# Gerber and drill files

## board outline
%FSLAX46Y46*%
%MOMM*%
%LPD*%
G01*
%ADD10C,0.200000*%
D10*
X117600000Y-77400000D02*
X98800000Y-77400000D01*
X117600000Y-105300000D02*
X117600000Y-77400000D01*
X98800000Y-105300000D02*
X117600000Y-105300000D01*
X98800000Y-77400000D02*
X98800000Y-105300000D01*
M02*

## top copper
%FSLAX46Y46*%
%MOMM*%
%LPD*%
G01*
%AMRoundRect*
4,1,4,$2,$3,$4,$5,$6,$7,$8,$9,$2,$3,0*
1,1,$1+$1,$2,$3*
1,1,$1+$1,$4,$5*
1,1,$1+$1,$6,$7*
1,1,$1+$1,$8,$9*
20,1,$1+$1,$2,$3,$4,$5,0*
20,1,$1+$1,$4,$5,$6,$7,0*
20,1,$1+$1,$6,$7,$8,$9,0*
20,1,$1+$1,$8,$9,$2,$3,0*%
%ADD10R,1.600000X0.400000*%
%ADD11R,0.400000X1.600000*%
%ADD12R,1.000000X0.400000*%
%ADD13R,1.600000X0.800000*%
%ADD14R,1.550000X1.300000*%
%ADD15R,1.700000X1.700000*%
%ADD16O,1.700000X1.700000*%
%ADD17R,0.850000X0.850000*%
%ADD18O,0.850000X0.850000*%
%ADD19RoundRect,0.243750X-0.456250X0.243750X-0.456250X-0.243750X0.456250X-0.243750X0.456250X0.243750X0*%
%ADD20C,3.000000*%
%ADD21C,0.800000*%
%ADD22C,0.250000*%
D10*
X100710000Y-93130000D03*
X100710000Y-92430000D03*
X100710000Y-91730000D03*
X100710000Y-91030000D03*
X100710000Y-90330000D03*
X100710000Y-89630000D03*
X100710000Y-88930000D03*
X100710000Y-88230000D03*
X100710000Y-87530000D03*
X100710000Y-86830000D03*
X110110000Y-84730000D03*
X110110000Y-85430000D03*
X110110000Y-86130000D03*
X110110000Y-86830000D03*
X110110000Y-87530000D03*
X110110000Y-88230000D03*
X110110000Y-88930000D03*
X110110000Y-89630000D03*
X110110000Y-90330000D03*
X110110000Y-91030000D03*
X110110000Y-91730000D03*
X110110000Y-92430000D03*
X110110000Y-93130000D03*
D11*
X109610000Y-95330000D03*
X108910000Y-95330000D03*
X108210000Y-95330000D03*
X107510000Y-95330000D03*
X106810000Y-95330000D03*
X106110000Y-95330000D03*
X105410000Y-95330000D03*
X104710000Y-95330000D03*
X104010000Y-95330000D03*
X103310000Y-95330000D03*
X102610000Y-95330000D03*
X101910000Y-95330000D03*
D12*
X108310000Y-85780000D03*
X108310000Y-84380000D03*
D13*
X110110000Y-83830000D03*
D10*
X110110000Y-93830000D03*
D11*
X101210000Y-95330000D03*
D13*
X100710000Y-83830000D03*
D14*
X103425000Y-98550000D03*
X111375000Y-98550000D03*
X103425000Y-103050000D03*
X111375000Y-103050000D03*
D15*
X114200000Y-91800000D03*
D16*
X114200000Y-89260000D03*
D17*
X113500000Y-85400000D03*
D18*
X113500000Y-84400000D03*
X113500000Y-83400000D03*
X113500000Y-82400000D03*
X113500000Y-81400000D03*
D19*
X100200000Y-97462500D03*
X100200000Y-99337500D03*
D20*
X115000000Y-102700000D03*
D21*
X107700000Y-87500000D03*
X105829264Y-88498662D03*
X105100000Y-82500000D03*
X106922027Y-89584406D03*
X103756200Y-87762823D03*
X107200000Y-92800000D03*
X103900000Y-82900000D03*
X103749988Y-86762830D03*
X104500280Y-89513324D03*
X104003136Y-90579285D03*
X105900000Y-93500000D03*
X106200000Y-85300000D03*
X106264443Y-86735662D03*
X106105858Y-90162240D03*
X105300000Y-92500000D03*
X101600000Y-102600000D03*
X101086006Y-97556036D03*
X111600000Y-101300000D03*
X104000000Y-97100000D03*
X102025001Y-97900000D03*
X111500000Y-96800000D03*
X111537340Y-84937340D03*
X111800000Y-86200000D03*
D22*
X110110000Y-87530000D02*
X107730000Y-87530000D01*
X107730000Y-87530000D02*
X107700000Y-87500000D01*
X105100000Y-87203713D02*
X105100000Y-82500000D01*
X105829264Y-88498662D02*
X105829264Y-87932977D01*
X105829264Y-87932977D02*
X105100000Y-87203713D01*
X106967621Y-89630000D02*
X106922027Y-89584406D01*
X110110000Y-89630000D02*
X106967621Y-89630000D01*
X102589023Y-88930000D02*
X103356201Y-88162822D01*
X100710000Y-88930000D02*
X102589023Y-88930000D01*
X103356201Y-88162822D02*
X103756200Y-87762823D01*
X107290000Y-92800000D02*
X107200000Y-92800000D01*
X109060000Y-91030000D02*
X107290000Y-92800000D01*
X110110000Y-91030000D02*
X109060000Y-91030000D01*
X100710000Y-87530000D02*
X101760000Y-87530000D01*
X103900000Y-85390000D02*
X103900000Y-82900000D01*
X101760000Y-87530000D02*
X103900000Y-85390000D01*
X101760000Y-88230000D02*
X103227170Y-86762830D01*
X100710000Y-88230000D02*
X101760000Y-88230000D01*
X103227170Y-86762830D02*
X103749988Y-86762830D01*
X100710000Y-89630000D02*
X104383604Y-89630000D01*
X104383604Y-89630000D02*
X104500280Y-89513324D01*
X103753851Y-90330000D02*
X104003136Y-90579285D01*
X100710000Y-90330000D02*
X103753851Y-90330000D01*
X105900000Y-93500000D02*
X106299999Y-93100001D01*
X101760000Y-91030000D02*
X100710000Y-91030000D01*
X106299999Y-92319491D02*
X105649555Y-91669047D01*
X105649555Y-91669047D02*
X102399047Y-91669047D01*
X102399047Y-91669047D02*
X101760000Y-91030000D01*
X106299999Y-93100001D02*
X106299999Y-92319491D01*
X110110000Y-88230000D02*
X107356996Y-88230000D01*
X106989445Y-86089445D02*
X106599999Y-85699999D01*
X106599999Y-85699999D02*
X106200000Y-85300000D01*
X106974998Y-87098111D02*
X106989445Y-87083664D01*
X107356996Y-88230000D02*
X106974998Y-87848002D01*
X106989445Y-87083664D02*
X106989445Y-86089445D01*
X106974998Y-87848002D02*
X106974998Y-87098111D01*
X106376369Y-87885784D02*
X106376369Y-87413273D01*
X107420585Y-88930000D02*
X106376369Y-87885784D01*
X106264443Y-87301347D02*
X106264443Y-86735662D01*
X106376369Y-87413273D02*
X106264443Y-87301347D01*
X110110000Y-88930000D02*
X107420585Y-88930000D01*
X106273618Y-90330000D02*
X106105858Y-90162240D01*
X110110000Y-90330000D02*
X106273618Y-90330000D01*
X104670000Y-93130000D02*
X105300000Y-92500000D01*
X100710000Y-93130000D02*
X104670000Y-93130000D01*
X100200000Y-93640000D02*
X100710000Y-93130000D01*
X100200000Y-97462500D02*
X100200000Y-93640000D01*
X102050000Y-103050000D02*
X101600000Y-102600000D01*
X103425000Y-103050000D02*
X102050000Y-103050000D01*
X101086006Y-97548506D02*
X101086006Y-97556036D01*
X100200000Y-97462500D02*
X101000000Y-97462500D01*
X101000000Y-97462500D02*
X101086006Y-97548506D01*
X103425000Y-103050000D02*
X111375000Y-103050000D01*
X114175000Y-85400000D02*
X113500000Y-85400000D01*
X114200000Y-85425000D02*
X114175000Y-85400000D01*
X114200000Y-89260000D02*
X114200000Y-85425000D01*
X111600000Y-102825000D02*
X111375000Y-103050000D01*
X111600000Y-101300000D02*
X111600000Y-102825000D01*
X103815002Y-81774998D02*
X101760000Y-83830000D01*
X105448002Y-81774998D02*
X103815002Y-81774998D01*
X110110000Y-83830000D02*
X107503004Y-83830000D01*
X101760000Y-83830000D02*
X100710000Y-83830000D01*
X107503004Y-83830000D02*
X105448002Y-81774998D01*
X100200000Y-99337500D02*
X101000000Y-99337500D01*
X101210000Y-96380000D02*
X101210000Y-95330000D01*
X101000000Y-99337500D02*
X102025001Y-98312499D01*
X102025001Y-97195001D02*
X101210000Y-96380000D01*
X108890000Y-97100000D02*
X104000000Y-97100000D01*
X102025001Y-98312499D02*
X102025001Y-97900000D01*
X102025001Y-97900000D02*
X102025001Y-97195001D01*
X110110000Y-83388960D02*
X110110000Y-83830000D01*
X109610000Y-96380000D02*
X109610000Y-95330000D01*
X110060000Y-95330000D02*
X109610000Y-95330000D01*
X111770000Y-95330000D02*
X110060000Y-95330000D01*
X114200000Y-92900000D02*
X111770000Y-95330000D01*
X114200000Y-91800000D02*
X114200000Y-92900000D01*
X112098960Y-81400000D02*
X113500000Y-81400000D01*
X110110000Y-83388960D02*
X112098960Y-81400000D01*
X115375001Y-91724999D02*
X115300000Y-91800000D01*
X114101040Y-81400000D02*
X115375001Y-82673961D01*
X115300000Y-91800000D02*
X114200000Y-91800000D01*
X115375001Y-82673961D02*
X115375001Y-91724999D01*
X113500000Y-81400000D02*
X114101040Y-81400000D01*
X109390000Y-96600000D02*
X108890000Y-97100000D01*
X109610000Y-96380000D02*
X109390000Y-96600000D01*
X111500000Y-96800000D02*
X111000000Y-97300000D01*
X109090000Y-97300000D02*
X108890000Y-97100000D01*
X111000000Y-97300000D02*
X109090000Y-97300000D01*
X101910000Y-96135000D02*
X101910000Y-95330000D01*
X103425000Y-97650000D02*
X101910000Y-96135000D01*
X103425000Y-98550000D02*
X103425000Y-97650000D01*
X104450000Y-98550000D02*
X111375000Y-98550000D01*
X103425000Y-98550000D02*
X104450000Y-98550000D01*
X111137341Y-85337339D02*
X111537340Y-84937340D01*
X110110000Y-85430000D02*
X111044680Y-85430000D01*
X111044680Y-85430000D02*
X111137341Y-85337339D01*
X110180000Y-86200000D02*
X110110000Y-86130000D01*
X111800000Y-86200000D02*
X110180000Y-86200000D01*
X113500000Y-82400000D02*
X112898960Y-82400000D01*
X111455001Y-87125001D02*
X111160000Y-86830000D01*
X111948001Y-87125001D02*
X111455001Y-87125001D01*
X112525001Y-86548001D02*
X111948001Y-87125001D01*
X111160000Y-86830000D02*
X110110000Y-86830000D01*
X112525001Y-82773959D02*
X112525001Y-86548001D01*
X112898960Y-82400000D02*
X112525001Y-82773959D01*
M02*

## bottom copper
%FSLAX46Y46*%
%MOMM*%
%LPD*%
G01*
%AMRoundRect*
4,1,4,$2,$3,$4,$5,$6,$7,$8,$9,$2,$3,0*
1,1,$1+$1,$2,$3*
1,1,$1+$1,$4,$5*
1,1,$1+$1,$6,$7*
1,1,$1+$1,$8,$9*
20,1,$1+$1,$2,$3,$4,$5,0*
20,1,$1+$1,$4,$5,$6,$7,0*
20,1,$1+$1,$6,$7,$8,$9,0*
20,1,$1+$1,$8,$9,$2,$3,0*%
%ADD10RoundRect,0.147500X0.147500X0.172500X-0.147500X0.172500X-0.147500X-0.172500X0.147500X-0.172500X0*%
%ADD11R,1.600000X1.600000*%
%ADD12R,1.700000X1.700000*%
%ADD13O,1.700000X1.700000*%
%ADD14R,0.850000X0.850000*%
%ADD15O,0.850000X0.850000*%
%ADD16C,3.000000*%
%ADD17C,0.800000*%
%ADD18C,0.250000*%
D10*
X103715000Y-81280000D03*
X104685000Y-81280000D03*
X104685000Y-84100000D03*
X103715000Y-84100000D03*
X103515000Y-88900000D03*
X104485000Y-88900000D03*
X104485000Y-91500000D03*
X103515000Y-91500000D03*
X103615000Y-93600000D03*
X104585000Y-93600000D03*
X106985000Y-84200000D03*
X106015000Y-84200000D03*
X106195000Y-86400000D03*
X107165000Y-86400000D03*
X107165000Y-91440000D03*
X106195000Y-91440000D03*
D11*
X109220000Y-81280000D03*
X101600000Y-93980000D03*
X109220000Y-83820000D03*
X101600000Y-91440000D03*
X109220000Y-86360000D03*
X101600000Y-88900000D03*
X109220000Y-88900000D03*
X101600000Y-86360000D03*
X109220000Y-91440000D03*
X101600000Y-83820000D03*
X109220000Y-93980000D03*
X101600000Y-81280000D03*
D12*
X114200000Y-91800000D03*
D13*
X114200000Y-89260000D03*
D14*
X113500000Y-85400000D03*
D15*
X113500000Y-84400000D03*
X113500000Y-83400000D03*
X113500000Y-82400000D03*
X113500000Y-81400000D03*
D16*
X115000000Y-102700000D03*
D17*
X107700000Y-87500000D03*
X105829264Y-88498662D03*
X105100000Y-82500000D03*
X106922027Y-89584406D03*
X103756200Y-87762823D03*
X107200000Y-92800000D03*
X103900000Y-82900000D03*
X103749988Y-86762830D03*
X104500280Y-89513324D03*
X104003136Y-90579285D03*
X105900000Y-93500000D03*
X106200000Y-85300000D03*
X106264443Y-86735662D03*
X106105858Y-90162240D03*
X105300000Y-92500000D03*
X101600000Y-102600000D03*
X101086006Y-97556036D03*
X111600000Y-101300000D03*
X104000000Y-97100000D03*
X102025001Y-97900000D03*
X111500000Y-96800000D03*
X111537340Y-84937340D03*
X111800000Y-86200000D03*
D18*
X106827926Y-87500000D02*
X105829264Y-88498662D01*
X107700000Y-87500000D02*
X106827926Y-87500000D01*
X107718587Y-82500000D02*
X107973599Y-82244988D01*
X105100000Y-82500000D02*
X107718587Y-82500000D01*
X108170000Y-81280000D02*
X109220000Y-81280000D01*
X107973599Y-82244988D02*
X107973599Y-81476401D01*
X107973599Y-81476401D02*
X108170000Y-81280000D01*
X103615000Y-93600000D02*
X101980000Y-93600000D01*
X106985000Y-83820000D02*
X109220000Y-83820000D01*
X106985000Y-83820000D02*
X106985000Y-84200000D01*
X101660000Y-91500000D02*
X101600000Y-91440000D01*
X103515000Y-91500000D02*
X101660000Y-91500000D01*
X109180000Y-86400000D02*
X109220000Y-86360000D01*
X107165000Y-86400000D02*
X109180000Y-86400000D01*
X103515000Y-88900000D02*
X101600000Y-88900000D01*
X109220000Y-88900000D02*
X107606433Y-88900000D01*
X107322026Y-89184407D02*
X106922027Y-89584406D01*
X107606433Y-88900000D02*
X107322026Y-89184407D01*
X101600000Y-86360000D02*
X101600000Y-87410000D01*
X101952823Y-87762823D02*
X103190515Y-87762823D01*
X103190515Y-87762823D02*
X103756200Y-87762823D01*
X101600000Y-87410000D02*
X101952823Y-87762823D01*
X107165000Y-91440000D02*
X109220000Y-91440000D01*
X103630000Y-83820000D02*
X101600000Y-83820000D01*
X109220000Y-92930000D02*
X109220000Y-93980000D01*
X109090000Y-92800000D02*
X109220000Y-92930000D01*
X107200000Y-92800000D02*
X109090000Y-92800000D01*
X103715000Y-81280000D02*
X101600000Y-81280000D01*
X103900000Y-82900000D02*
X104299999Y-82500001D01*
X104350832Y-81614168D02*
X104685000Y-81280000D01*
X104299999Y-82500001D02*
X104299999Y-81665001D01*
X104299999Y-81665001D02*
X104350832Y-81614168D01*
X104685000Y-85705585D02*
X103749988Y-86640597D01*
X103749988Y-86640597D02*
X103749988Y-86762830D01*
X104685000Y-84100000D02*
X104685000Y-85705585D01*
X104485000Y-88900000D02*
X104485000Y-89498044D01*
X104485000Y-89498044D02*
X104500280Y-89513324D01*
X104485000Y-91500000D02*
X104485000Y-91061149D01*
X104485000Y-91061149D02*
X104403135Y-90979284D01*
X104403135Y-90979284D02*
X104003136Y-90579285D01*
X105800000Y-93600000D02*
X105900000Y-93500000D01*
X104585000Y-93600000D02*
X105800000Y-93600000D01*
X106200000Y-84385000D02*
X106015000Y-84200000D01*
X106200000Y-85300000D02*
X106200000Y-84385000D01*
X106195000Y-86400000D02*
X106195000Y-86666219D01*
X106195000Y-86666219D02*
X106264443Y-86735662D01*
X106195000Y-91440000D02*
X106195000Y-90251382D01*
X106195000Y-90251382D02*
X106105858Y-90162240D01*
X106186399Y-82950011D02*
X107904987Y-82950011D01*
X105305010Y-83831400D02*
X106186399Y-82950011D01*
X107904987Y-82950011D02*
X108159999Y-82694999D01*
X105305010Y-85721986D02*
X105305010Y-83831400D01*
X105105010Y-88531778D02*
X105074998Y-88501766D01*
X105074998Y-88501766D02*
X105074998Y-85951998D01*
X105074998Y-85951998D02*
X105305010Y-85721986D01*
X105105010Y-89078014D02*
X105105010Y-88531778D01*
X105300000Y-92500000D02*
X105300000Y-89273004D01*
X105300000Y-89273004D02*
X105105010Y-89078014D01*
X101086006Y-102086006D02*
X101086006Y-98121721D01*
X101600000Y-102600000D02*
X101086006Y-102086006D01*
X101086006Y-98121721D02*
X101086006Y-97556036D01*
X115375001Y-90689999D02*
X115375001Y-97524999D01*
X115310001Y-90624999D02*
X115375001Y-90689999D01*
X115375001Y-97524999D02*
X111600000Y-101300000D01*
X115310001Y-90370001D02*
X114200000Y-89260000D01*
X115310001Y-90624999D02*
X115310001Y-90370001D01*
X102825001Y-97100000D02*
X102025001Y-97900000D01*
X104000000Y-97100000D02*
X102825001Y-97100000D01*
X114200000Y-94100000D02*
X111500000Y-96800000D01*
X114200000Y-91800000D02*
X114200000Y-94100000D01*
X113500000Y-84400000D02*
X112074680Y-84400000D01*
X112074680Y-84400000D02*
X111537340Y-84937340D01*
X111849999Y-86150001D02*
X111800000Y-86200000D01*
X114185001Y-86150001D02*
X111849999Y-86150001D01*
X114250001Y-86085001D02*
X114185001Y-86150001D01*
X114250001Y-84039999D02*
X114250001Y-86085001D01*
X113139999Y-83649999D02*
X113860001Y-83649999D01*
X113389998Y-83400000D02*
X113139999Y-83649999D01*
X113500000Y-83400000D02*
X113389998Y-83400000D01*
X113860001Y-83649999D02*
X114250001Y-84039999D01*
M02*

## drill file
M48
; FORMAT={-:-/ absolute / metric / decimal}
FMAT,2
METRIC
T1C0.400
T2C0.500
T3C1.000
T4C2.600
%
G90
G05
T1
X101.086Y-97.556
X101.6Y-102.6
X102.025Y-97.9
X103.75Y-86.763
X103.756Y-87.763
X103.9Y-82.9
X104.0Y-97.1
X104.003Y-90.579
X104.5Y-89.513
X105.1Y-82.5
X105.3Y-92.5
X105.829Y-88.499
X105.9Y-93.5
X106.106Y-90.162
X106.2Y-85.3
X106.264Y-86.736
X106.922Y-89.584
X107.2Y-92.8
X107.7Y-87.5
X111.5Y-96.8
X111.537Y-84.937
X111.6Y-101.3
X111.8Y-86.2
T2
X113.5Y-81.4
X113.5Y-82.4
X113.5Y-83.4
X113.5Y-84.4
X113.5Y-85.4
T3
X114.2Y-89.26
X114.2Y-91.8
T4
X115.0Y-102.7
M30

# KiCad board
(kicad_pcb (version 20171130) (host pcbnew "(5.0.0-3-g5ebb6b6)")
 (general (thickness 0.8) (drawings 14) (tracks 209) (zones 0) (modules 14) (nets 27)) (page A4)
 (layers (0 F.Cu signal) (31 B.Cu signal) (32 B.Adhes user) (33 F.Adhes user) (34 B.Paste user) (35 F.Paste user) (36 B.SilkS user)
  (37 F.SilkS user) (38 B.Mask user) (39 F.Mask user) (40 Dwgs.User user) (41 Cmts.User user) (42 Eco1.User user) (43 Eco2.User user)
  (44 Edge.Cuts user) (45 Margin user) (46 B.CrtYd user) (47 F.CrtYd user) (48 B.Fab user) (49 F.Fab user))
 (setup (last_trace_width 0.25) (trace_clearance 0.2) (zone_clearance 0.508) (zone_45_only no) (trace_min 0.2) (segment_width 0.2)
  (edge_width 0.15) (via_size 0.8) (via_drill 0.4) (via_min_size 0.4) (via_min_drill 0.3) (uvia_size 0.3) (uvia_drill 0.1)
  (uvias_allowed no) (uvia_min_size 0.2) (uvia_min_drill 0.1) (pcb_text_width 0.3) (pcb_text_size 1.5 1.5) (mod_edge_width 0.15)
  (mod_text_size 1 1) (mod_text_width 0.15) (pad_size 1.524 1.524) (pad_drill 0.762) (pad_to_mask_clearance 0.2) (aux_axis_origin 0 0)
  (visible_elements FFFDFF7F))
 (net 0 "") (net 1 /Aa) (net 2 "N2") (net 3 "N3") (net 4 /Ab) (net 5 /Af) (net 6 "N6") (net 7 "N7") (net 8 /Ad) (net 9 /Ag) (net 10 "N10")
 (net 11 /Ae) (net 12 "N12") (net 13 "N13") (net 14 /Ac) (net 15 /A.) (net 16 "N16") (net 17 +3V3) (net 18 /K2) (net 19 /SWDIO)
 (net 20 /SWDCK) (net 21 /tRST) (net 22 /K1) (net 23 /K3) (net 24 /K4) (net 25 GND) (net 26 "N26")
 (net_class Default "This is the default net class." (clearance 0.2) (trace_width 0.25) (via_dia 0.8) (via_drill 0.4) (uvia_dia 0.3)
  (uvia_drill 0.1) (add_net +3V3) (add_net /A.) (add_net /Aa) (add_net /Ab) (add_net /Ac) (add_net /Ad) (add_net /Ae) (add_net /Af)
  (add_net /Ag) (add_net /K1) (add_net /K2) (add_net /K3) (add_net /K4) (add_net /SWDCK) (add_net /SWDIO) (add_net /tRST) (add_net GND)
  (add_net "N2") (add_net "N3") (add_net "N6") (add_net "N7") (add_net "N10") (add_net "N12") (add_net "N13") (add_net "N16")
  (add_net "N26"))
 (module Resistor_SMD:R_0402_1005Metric (layer B.Cu) (at 104.2 81.28 180)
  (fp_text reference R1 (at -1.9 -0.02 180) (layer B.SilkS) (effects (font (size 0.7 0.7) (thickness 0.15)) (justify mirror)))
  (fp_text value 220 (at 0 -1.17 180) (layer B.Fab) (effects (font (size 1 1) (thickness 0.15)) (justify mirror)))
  (pad 2 smd roundrect (at 0.485 0 180) (size 0.59 0.64) (layers B.Cu B.Paste B.Mask) (roundrect_rratio 0.25) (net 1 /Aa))
  (pad 1 smd roundrect (at -0.485 0 180) (size 0.59 0.64) (layers B.Cu B.Paste B.Mask) (roundrect_rratio 0.25) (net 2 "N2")))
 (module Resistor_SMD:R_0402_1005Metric (layer B.Cu) (at 104.2 84.1 180)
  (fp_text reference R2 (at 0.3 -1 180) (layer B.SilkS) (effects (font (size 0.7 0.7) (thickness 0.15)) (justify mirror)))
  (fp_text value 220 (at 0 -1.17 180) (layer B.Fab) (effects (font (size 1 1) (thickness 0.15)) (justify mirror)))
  (pad 1 smd roundrect (at -0.485 0 180) (size 0.59 0.64) (layers B.Cu B.Paste B.Mask) (roundrect_rratio 0.25) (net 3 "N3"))
  (pad 2 smd roundrect (at 0.485 0 180) (size 0.59 0.64) (layers B.Cu B.Paste B.Mask) (roundrect_rratio 0.25) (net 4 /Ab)))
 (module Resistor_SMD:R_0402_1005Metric (layer B.Cu) (at 104 88.9 180)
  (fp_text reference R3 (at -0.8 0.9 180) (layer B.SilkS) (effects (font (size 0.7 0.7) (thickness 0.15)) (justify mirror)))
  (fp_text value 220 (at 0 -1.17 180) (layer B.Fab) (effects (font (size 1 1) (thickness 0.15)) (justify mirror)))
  (pad 2 smd roundrect (at 0.485 0 180) (size 0.59 0.64) (layers B.Cu B.Paste B.Mask) (roundrect_rratio 0.25) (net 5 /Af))
  (pad 1 smd roundrect (at -0.485 0 180) (size 0.59 0.64) (layers B.Cu B.Paste B.Mask) (roundrect_rratio 0.25) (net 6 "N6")))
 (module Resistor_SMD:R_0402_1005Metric (layer B.Cu) (at 104 91.5 180)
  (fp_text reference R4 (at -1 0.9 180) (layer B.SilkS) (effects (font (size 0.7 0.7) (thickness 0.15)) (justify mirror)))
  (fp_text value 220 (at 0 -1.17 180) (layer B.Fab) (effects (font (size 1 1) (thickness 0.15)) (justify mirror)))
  (pad 1 smd roundrect (at -0.485 0 180) (size 0.59 0.64) (layers B.Cu B.Paste B.Mask) (roundrect_rratio 0.25) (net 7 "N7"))
  (pad 2 smd roundrect (at 0.485 0 180) (size 0.59 0.64) (layers B.Cu B.Paste B.Mask) (roundrect_rratio 0.25) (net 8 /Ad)))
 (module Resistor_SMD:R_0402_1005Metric (layer B.Cu) (at 104.1 93.6 180)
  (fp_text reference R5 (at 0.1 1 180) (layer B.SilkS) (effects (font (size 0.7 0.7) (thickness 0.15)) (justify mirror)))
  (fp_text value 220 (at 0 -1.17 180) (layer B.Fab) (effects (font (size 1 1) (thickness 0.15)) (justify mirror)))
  (pad 2 smd roundrect (at 0.485 0 180) (size 0.59 0.64) (layers B.Cu B.Paste B.Mask) (roundrect_rratio 0.25) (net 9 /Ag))
  (pad 1 smd roundrect (at -0.485 0 180) (size 0.59 0.64) (layers B.Cu B.Paste B.Mask) (roundrect_rratio 0.25) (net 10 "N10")))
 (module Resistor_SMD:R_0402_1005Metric (layer B.Cu) (at 106.5 84.2 180)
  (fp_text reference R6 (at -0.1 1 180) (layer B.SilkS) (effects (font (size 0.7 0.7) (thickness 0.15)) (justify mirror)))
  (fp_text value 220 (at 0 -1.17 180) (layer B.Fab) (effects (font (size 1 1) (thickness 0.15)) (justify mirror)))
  (pad 1 smd roundrect (at -0.485 0 180) (size 0.59 0.64) (layers B.Cu B.Paste B.Mask) (roundrect_rratio 0.25) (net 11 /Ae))
  (pad 2 smd roundrect (at 0.485 0 180) (size 0.59 0.64) (layers B.Cu B.Paste B.Mask) (roundrect_rratio 0.25) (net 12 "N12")))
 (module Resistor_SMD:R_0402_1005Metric (layer B.Cu) (at 106.68 86.4 180)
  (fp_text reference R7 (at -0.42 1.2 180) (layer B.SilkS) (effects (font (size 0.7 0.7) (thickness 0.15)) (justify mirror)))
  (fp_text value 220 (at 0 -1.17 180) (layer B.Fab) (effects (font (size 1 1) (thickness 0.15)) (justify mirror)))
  (pad 2 smd roundrect (at 0.485 0 180) (size 0.59 0.64) (layers B.Cu B.Paste B.Mask) (roundrect_rratio 0.25) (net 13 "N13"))
  (pad 1 smd roundrect (at -0.485 0 180) (size 0.59 0.64) (layers B.Cu B.Paste B.Mask) (roundrect_rratio 0.25) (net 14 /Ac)))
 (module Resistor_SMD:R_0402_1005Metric (layer B.Cu) (at 106.68 91.44 180)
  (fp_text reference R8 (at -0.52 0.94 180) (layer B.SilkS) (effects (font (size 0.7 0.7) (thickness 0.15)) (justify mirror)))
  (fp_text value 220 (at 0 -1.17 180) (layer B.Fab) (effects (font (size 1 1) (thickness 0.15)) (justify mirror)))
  (pad 1 smd roundrect (at -0.485 0 180) (size 0.59 0.64) (layers B.Cu B.Paste B.Mask) (roundrect_rratio 0.25) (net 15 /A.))
  (pad 2 smd roundrect (at 0.485 0 180) (size 0.59 0.64) (layers B.Cu B.Paste B.Mask) (roundrect_rratio 0.25) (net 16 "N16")))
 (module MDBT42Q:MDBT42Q (layer F.Cu) (at 105.41 87.63)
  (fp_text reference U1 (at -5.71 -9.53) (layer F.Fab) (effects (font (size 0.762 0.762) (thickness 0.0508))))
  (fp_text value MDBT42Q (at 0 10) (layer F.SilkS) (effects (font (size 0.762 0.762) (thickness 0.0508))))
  (pad 11 smd rect (at -4.7 5.5) (size 1.6 0.4) (layers F.Cu F.Paste F.Mask) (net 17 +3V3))
  (pad 10 smd rect (at -4.7 4.8) (size 1.6 0.4) (layers F.Cu F.Paste F.Mask))
  (pad 9 smd rect (at -4.7 4.1) (size 1.6 0.4) (layers F.Cu F.Paste F.Mask))
  (pad 8 smd rect (at -4.7 3.4) (size 1.6 0.4) (layers F.Cu F.Paste F.Mask) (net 10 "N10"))
  (pad 7 smd rect (at -4.7 2.7) (size 1.6 0.4) (layers F.Cu F.Paste F.Mask) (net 7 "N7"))
  (pad 6 smd rect (at -4.7 2) (size 1.6 0.4) (layers F.Cu F.Paste F.Mask) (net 6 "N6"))
  (pad 5 smd rect (at -4.7 1.3) (size 1.6 0.4) (layers F.Cu F.Paste F.Mask) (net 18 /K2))
  (pad 4 smd rect (at -4.7 0.6) (size 1.6 0.4) (layers F.Cu F.Paste F.Mask) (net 3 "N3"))
  (pad 3 smd rect (at -4.7 -0.1) (size 1.6 0.4) (layers F.Cu F.Paste F.Mask) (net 2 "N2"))
  (pad 2 smd rect (at -4.7 -0.8) (size 1.6 0.4) (layers F.Cu F.Paste F.Mask))
  (pad 38 smd rect (at 4.7 -2.9 180) (size 1.6 0.4) (layers F.Cu F.Paste F.Mask))
  (pad 37 smd rect (at 4.7 -2.2 180) (size 1.6 0.4) (layers F.Cu F.Paste F.Mask) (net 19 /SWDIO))
  (pad 36 smd rect (at 4.7 -1.5 180) (size 1.6 0.4) (layers F.Cu F.Paste F.Mask) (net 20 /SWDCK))
  (pad 35 smd rect (at 4.7 -0.8 180) (size 1.6 0.4) (layers F.Cu F.Paste F.Mask) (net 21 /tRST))
  (pad 34 smd rect (at 4.7 -0.1 180) (size 1.6 0.4) (layers F.Cu F.Paste F.Mask) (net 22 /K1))
  (pad 33 smd rect (at 4.7 0.6 180) (size 1.6 0.4) (layers F.Cu F.Paste F.Mask) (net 12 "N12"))
  (pad 32 smd rect (at 4.7 1.3 180) (size 1.6 0.4) (layers F.Cu F.Paste F.Mask) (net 13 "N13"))
  (pad 31 smd rect (at 4.7 2 180) (size 1.6 0.4) (layers F.Cu F.Paste F.Mask) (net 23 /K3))
  (pad 30 smd rect (at 4.7 2.7 180) (size 1.6 0.4) (layers F.Cu F.Paste F.Mask) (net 16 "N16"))
  (pad 29 smd rect (at 4.7 3.4 180) (size 1.6 0.4) (layers F.Cu F.Paste F.Mask) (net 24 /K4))
  (pad 28 smd rect (at 4.7 4.1 180) (size 1.6 0.4) (layers F.Cu F.Paste F.Mask))
  (pad 27 smd rect (at 4.7 4.8 180) (size 1.6 0.4) (layers F.Cu F.Paste F.Mask))
  (pad 26 smd rect (at 4.7 5.5 180) (size 1.6 0.4) (layers F.Cu F.Paste F.Mask))
  (pad 24 smd rect (at 4.2 7.7 90) (size 1.6 0.4) (layers F.Cu F.Paste F.Mask) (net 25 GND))
  (pad 23 smd rect (at 3.5 7.7 90) (size 1.6 0.4) (layers F.Cu F.Paste F.Mask))
  (pad 22 smd rect (at 2.8 7.7 90) (size 1.6 0.4) (layers F.Cu F.Paste F.Mask))
  (pad 21 smd rect (at 2.1 7.7 90) (size 1.6 0.4) (layers F.Cu F.Paste F.Mask))
  (pad 20 smd rect (at 1.4 7.7 90) (size 1.6 0.4) (layers F.Cu F.Paste F.Mask))
  (pad 19 smd rect (at 0.7 7.7 90) (size 1.6 0.4) (layers F.Cu F.Paste F.Mask))
  (pad 18 smd rect (at 0 7.7 90) (size 1.6 0.4) (layers F.Cu F.Paste F.Mask))
  (pad 17 smd rect (at -0.7 7.7 90) (size 1.6 0.4) (layers F.Cu F.Paste F.Mask))
  (pad 16 smd rect (at -1.4 7.7 90) (size 1.6 0.4) (layers F.Cu F.Paste F.Mask))
  (pad 15 smd rect (at -2.1 7.7 90) (size 1.6 0.4) (layers F.Cu F.Paste F.Mask))
  (pad 14 smd rect (at -2.8 7.7 90) (size 1.6 0.4) (layers F.Cu F.Paste F.Mask))
  (pad 13 smd rect (at -3.5 7.7 90) (size 1.6 0.4) (layers F.Cu F.Paste F.Mask) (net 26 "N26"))
  (pad 41 smd rect (at 2.9 -1.85 180) (size 1 0.4) (layers F.Cu F.Paste F.Mask))
  (pad 40 smd rect (at 2.9 -3.25 180) (size 1 0.4) (layers F.Cu F.Paste F.Mask))
  (pad 39 smd rect (at 4.7 -3.8 180) (size 1.6 0.8) (layers F.Cu F.Paste F.Mask) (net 25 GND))
  (pad 25 smd rect (at 4.7 6.2 180) (size 1.6 0.4) (layers F.Cu F.Paste F.Mask))
  (pad 12 smd rect (at -4.2 7.7 90) (size 1.6 0.4) (layers F.Cu F.Paste F.Mask) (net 25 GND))
  (pad 1 smd rect (at -4.7 -3.8) (size 1.6 0.8) (layers F.Cu F.Paste F.Mask) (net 25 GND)))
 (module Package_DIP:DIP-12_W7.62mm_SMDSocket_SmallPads (layer B.Cu) (at 105.41 87.63 180)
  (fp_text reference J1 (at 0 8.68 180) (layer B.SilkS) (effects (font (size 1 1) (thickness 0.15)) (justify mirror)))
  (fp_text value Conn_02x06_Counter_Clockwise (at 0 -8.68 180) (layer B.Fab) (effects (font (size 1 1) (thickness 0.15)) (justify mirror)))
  (pad 1 smd rect (at -3.81 6.35 180) (size 1.6 1.6) (layers B.Cu B.Paste B.Mask) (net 22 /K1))
  (pad 7 smd rect (at 3.81 -6.35 180) (size 1.6 1.6) (layers B.Cu B.Paste B.Mask) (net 9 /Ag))
  (pad 2 smd rect (at -3.81 3.81 180) (size 1.6 1.6) (layers B.Cu B.Paste B.Mask) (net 11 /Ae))
  (pad 8 smd rect (at 3.81 -3.81 180) (size 1.6 1.6) (layers B.Cu B.Paste B.Mask) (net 8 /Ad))
  (pad 3 smd rect (at -3.81 1.27 180) (size 1.6 1.6) (layers B.Cu B.Paste B.Mask) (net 14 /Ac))
  (pad 9 smd rect (at 3.81 -1.27 180) (size 1.6 1.6) (layers B.Cu B.Paste B.Mask) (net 5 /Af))
  (pad 4 smd rect (at -3.81 -1.27 180) (size 1.6 1.6) (layers B.Cu B.Paste B.Mask) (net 23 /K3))
  (pad 10 smd rect (at 3.81 1.27 180) (size 1.6 1.6) (layers B.Cu B.Paste B.Mask) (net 18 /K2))
  (pad 5 smd rect (at -3.81 -3.81 180) (size 1.6 1.6) (layers B.Cu B.Paste B.Mask) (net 15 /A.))
  (pad 11 smd rect (at 3.81 3.81 180) (size 1.6 1.6) (layers B.Cu B.Paste B.Mask) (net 4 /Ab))
  (pad 6 smd rect (at -3.81 -6.35 180) (size 1.6 1.6) (layers B.Cu B.Paste B.Mask) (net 24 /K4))
  (pad 12 smd rect (at 3.81 6.35 180) (size 1.6 1.6) (layers B.Cu B.Paste B.Mask) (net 1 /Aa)))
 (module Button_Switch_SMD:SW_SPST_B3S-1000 (layer F.Cu) (at 107.4 100.8)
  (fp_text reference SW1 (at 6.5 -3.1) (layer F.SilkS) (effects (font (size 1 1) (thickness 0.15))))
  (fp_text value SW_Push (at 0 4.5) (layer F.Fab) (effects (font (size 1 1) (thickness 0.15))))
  (pad 1 smd rect (at -3.975 -2.25) (size 1.55 1.3) (layers F.Cu F.Paste F.Mask) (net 26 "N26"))
  (pad 1 smd rect (at 3.975 -2.25) (size 1.55 1.3) (layers F.Cu F.Paste F.Mask) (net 26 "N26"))
  (pad 2 smd rect (at -3.975 2.25) (size 1.55 1.3) (layers F.Cu F.Paste F.Mask) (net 17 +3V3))
  (pad 2 smd rect (at 3.975 2.25) (size 1.55 1.3) (layers F.Cu F.Paste F.Mask) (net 17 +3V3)))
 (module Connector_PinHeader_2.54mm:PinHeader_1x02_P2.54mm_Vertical (layer F.Cu) (at 114.2 91.8 180)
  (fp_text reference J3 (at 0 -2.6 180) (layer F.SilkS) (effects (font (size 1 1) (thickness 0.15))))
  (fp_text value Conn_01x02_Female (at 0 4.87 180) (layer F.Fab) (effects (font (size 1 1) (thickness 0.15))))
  (pad 1 thru_hole rect (at 0 0 180) (size 1.7 1.7) (drill 1) (layers *.Cu *.Mask) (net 25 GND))
  (pad 2 thru_hole oval (at 0 2.54 180) (size 1.7 1.7) (drill 1) (layers *.Cu *.Mask) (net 17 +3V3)))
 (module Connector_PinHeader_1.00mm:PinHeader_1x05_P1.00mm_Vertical (layer F.Cu) (at 113.5 85.4 180)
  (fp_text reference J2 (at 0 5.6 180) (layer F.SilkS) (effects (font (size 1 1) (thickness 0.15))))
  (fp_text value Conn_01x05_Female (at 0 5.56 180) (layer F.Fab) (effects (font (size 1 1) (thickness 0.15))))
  (pad 1 thru_hole rect (at 0 0 180) (size 0.85 0.85) (drill 0.5) (layers *.Cu *.Mask) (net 17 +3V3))
  (pad 2 thru_hole oval (at 0 1 180) (size 0.85 0.85) (drill 0.5) (layers *.Cu *.Mask) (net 19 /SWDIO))
  (pad 3 thru_hole oval (at 0 2 180) (size 0.85 0.85) (drill 0.5) (layers *.Cu *.Mask) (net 20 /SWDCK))
  (pad 4 thru_hole oval (at 0 3 180) (size 0.85 0.85) (drill 0.5) (layers *.Cu *.Mask) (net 21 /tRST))
  (pad 5 thru_hole oval (at 0 4 180) (size 0.85 0.85) (drill 0.5) (layers *.Cu *.Mask) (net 25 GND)))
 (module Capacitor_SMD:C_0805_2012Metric (layer F.Cu) (at 100.2 98.4 270)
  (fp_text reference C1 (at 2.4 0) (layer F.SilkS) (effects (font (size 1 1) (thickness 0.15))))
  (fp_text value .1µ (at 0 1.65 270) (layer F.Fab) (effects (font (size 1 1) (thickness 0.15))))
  (pad 1 smd roundrect (at -0.9375 0 270) (size 0.975 1.4) (layers F.Cu F.Paste F.Mask) (roundrect_rratio 0.25) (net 17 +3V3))
  (pad 2 smd roundrect (at 0.9375 0 270) (size 0.975 1.4) (layers F.Cu F.Paste F.Mask) (roundrect_rratio 0.25) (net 25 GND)))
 (gr_line (start 117.6 77.4) (end 98.8 77.4) (layer Edge.Cuts) (width 0.2))
 (gr_line (start 117.6 105.3) (end 117.6 77.4) (layer Edge.Cuts) (width 0.2))
 (gr_line (start 98.8 105.3) (end 117.6 105.3) (layer Edge.Cuts) (width 0.2))
 (gr_line (start 98.8 77.4) (end 98.8 105.3) (layer Edge.Cuts) (width 0.2))
 (via (at 115 102.7) (size 3) (drill 2.6) (layers F.Cu B.Cu) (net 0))
 (via (at 107.7 87.5) (size 0.8) (drill 0.4) (layers F.Cu B.Cu) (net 22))
 (segment (start 110.11 87.53) (end 107.73 87.53) (width 0.25) (layer F.Cu) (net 22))
 (segment (start 107.73 87.53) (end 107.7 87.5) (width 0.25) (layer F.Cu) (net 22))
 (segment (start 106.827926 87.5) (end 105.829264 88.498662) (width 0.25) (layer B.Cu) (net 22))
 (via (at 105.829264 88.498662) (size 0.8) (drill 0.4) (layers F.Cu B.Cu) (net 22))
 (segment (start 107.7 87.5) (end 106.827926 87.5) (width 0.25) (layer B.Cu) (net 22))
 (via (at 105.1 82.5) (size 0.8) (drill 0.4) (layers F.Cu B.Cu) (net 22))
 (segment (start 105.1 87.203713) (end 105.1 82.5) (width 0.25) (layer F.Cu) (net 22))
 (segment (start 105.829264 88.498662) (end 105.829264 87.932977) (width 0.25) (layer F.Cu) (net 22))
 (segment (start 105.829264 87.932977) (end 105.1 87.203713) (width 0.25) (layer F.Cu) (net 22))
 (segment (start 107.718587 82.5) (end 107.973599 82.244988) (width 0.25) (layer B.Cu) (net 22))
 (segment (start 105.1 82.5) (end 107.718587 82.5) (width 0.25) (layer B.Cu) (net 22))
 (segment (start 108.17 81.28) (end 109.22 81.28) (width 0.25) (layer B.Cu) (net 22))
 (segment (start 107.973599 82.244988) (end 107.973599 81.476401) (width 0.25) (layer B.Cu) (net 22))
 (segment (start 107.973599 81.476401) (end 108.17 81.28) (width 0.25) (layer B.Cu) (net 22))
 (segment (start 103.615 93.6) (end 101.98 93.6) (width 0.25) (layer B.Cu) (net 9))
 (segment (start 106.985 83.82) (end 109.22 83.82) (width 0.25) (layer B.Cu) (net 11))
 (segment (start 106.985 83.82) (end 106.985 84.2) (width 0.25) (layer B.Cu) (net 11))
 (segment (start 101.66 91.5) (end 101.6 91.44) (width 0.25) (layer B.Cu) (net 8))
 (segment (start 103.515 91.5) (end 101.66 91.5) (width 0.25) (layer B.Cu) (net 8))
 (segment (start 109.18 86.4) (end 109.22 86.36) (width 0.25) (layer B.Cu) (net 14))
 (segment (start 107.165 86.4) (end 109.18 86.4) (width 0.25) (layer B.Cu) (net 14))
 (segment (start 103.515 88.9) (end 101.6 88.9) (width 0.25) (layer B.Cu) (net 5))
 (segment (start 106.967621 89.63) (end 106.922027 89.584406) (width 0.25) (layer F.Cu) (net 23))
 (segment (start 109.22 88.9) (end 107.606433 88.9) (width 0.25) (layer B.Cu) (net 23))
 (segment (start 110.11 89.63) (end 106.967621 89.63) (width 0.25) (layer F.Cu) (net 23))
 (segment (start 107.322026 89.184407) (end 106.922027 89.584406) (width 0.25) (layer B.Cu) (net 23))
 (via (at 106.922027 89.584406) (size 0.8) (drill 0.4) (layers F.Cu B.Cu) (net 23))
 (segment (start 107.606433 88.9) (end 107.322026 89.184407) (width 0.25) (layer B.Cu) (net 23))
 (segment (start 101.6 86.36) (end 101.6 87.41) (width 0.25) (layer B.Cu) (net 18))
 (segment (start 102.589023 88.93) (end 103.356201 88.162822) (width 0.25) (layer F.Cu) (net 18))
 (via (at 103.7562 87.762823) (size 0.8) (drill 0.4) (layers F.Cu B.Cu) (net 18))
 (segment (start 101.952823 87.762823) (end 103.190515 87.762823) (width 0.25) (layer B.Cu) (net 18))
 (segment (start 100.71 88.93) (end 102.589023 88.93) (width 0.25) (layer F.Cu) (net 18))
 (segment (start 103.356201 88.162822) (end 103.7562 87.762823) (width 0.25) (layer F.Cu) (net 18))
 (segment (start 103.190515 87.762823) (end 103.7562 87.762823) (width 0.25) (layer B.Cu) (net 18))
 (segment (start 101.6 87.41) (end 101.952823 87.762823) (width 0.25) (layer B.Cu) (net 18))
 (segment (start 107.165 91.44) (end 109.22 91.44) (width 0.25) (layer B.Cu) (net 15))
 (segment (start 103.63 83.82) (end 101.6 83.82) (width 0.25) (layer B.Cu) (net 4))
 (via (at 107.2 92.8) (size 0.8) (drill 0.4) (layers F.Cu B.Cu) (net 24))
 (segment (start 107.29 92.8) (end 107.2 92.8) (width 0.25) (layer F.Cu) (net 24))
 (segment (start 109.06 91.03) (end 107.29 92.8) (width 0.25) (layer F.Cu) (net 24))
 (segment (start 110.11 91.03) (end 109.06 91.03) (width 0.25) (layer F.Cu) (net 24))
 (segment (start 109.22 92.93) (end 109.22 93.98) (width 0.25) (layer B.Cu) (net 24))
 (segment (start 109.09 92.8) (end 109.22 92.93) (width 0.25) (layer B.Cu) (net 24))
 (segment (start 107.2 92.8) (end 109.09 92.8) (width 0.25) (layer B.Cu) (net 24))
 (segment (start 103.715 81.28) (end 101.6 81.28) (width 0.25) (layer B.Cu) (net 1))
 (via (at 103.9 82.9) (size 0.8) (drill 0.4) (layers F.Cu B.Cu) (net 2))
 (segment (start 100.71 87.53) (end 101.76 87.53) (width 0.25) (layer F.Cu) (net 2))
 (segment (start 103.9 85.39) (end 103.9 82.9) (width 0.25) (layer F.Cu) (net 2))
 (segment (start 101.76 87.53) (end 103.9 85.39) (width 0.25) (layer F.Cu) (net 2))
 (segment (start 103.9 82.9) (end 104.299999 82.500001) (width 0.25) (layer B.Cu) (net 2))
 (segment (start 104.350832 81.614168) (end 104.685 81.28) (width 0.25) (layer B.Cu) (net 2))
 (segment (start 104.299999 82.500001) (end 104.299999 81.665001) (width 0.25) (layer B.Cu) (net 2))
 (segment (start 104.299999 81.665001) (end 104.350832 81.614168) (width 0.25) (layer B.Cu) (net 2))
 (via (at 103.749988 86.76283) (size 0.8) (drill 0.4) (layers F.Cu B.Cu) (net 3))
 (segment (start 104.685 85.705585) (end 103.749988 86.640597) (width 0.25) (layer B.Cu) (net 3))
 (segment (start 101.76 88.23) (end 103.22717 86.76283) (width 0.25) (layer F.Cu) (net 3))
 (segment (start 100.71 88.23) (end 101.76 88.23) (width 0.25) (layer F.Cu) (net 3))
 (segment (start 103.749988 86.640597) (end 103.749988 86.76283) (width 0.25) (layer B.Cu) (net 3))
 (segment (start 103.22717 86.76283) (end 103.749988 86.76283) (width 0.25) (layer F.Cu) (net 3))
 (segment (start 104.685 84.1) (end 104.685 85.705585) (width 0.25) (layer B.Cu) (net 3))
 (segment (start 100.71 89.63) (end 104.383604 89.63) (width 0.25) (layer F.Cu) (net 6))
 (segment (start 104.485 88.9) (end 104.485 89.498044) (width 0.25) (layer B.Cu) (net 6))
 (segment (start 104.485 89.498044) (end 104.50028 89.513324) (width 0.25) (layer B.Cu) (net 6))
 (via (at 104.50028 89.513324) (size 0.8) (drill 0.4) (layers F.Cu B.Cu) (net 6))
 (segment (start 104.383604 89.63) (end 104.50028 89.513324) (width 0.25) (layer F.Cu) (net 6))
 (segment (start 103.753851 90.33) (end 104.003136 90.579285) (width 0.25) (layer F.Cu) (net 7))
 (segment (start 104.485 91.5) (end 104.485 91.061149) (width 0.25) (layer B.Cu) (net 7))
 (segment (start 104.485 91.061149) (end 104.403135 90.979284) (width 0.25) (layer B.Cu) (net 7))
 (via (at 104.003136 90.579285) (size 0.8) (drill 0.4) (layers F.Cu B.Cu) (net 7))
 (segment (start 104.403135 90.979284) (end 104.003136 90.579285) (width 0.25) (layer B.Cu) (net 7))
 (segment (start 100.71 90.33) (end 103.753851 90.33) (width 0.25) (layer F.Cu) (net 7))
 (segment (start 105.8 93.6) (end 105.9 93.5) (width 0.25) (layer B.Cu) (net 10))
 (via (at 105.9 93.5) (size 0.8) (drill 0.4) (layers F.Cu B.Cu) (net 10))
 (segment (start 104.585 93.6) (end 105.8 93.6) (width 0.25) (layer B.Cu) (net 10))
 (segment (start 105.9 93.5) (end 106.299999 93.100001) (width 0.25) (layer F.Cu) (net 10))
 (segment (start 101.76 91.03) (end 100.71 91.03) (width 0.25) (layer F.Cu) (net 10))
 (segment (start 106.299999 92.319491) (end 105.649555 91.669047) (width 0.25) (layer F.Cu) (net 10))
 (segment (start 105.649555 91.669047) (end 102.399047 91.669047) (width 0.25) (layer F.Cu) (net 10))
 (segment (start 102.399047 91.669047) (end 101.76 91.03) (width 0.25) (layer F.Cu) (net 10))
 (segment (start 106.299999 93.100001) (end 106.299999 92.319491) (width 0.25) (layer F.Cu) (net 10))
 (via (at 106.2 85.3) (size 0.8) (drill 0.4) (layers F.Cu B.Cu) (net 12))
 (segment (start 106.2 84.385) (end 106.015 84.2) (width 0.25) (layer B.Cu) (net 12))
 (segment (start 106.2 85.3) (end 106.2 84.385) (width 0.25) (layer B.Cu) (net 12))
 (segment (start 110.11 88.23) (end 107.356996 88.23) (width 0.25) (layer F.Cu) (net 12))
 (segment (start 106.989445 86.089445) (end 106.599999 85.699999) (width 0.25) (layer F.Cu) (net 12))
 (segment (start 106.599999 85.699999) (end 106.2 85.3) (width 0.25) (layer F.Cu) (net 12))
 (segment (start 106.974998 87.098111) (end 106.989445 87.083664) (width 0.25) (layer F.Cu) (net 12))
 (segment (start 107.356996 88.23) (end 106.974998 87.848002) (width 0.25) (layer F.Cu) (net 12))
 (segment (start 106.989445 87.083664) (end 106.989445 86.089445) (width 0.25) (layer F.Cu) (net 12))
 (segment (start 106.974998 87.848002) (end 106.974998 87.098111) (width 0.25) (layer F.Cu) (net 12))
 (segment (start 106.376369 87.885784) (end 106.376369 87.413273) (width 0.25) (layer F.Cu) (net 13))
 (segment (start 107.420585 88.93) (end 106.376369 87.885784) (width 0.25) (layer F.Cu) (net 13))
 (segment (start 106.264443 87.301347) (end 106.264443 86.735662) (width 0.25) (layer F.Cu) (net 13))
 (via (at 106.264443 86.735662) (size 0.8) (drill 0.4) (layers F.Cu B.Cu) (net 13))
 (segment (start 106.195 86.4) (end 106.195 86.666219) (width 0.25) (layer B.Cu) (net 13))
 (segment (start 106.195 86.666219) (end 106.264443 86.735662) (width 0.25) (layer B.Cu) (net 13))
 (segment (start 106.376369 87.413273) (end 106.264443 87.301347) (width 0.25) (layer F.Cu) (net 13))
 (segment (start 110.11 88.93) (end 107.420585 88.93) (width 0.25) (layer F.Cu) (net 13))
 (via (at 106.105858 90.16224) (size 0.8) (drill 0.4) (layers F.Cu B.Cu) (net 16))
 (segment (start 106.273618 90.33) (end 106.105858 90.16224) (width 0.25) (layer F.Cu) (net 16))
 (segment (start 106.195 91.44) (end 106.195 90.251382) (width 0.25) (layer B.Cu) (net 16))
 (segment (start 106.195 90.251382) (end 106.105858 90.16224) (width 0.25) (layer B.Cu) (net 16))
 (segment (start 110.11 90.33) (end 106.273618 90.33) (width 0.25) (layer F.Cu) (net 16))
 (via (at 105.3 92.5) (size 0.8) (drill 0.4) (layers F.Cu B.Cu) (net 17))
 (segment (start 104.67 93.13) (end 105.3 92.5) (width 0.25) (layer F.Cu) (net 17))
 (segment (start 100.71 93.13) (end 104.67 93.13) (width 0.25) (layer F.Cu) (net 17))
 (segment (start 106.186399 82.950011) (end 107.904987 82.950011) (width 0.25) (layer B.Cu) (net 17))
 (segment (start 105.30501 83.8314) (end 106.186399 82.950011) (width 0.25) (layer B.Cu) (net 17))
 (segment (start 107.904987 82.950011) (end 108.159999 82.694999) (width 0.25) (layer B.Cu) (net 17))
 (segment (start 105.30501 85.721986) (end 105.30501 83.8314) (width 0.25) (layer B.Cu) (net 17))
 (segment (start 105.10501 88.531778) (end 105.074998 88.501766) (width 0.25) (layer B.Cu) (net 17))
 (segment (start 105.074998 88.501766) (end 105.074998 85.951998) (width 0.25) (layer B.Cu) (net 17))
 (segment (start 105.074998 85.951998) (end 105.30501 85.721986) (width 0.25) (layer B.Cu) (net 17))
 (segment (start 105.10501 89.078014) (end 105.10501 88.531778) (width 0.25) (layer B.Cu) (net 17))
 (segment (start 105.3 92.5) (end 105.3 89.273004) (width 0.25) (layer B.Cu) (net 17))
 (segment (start 105.3 89.273004) (end 105.10501 89.078014) (width 0.25) (layer B.Cu) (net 17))
 (segment (start 100.2 93.64) (end 100.71 93.13) (width 0.25) (layer F.Cu) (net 17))
 (segment (start 100.2 97.4625) (end 100.2 93.64) (width 0.25) (layer F.Cu) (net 17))
 (via (at 101.6 102.6) (size 0.8) (drill 0.4) (layers F.Cu B.Cu) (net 17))
 (segment (start 102.05 103.05) (end 101.6 102.6) (width 0.25) (layer F.Cu) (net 17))
 (segment (start 103.425 103.05) (end 102.05 103.05) (width 0.25) (layer F.Cu) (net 17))
 (via (at 101.086006 97.556036) (size 0.8) (drill 0.4) (layers F.Cu B.Cu) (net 17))
 (segment (start 101.086006 97.548506) (end 101.086006 97.556036) (width 0.25) (layer F.Cu) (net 17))
 (segment (start 100.2 97.4625) (end 101 97.4625) (width 0.25) (layer F.Cu) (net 17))
 (segment (start 101 97.4625) (end 101.086006 97.548506) (width 0.25) (layer F.Cu) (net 17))
 (segment (start 101.086006 102.086006) (end 101.086006 98.121721) (width 0.25) (layer B.Cu) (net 17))
 (segment (start 101.6 102.6) (end 101.086006 102.086006) (width 0.25) (layer B.Cu) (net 17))
 (segment (start 101.086006 98.121721) (end 101.086006 97.556036) (width 0.25) (layer B.Cu) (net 17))
 (segment (start 103.425 103.05) (end 111.375 103.05) (width 0.25) (layer F.Cu) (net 17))
 (segment (start 114.175 85.4) (end 113.5 85.4) (width 0.25) (layer F.Cu) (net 17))
 (segment (start 114.2 85.425) (end 114.175 85.4) (width 0.25) (layer F.Cu) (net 17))
 (segment (start 114.2 89.26) (end 114.2 85.425) (width 0.25) (layer F.Cu) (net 17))
 (via (at 111.6 101.3) (size 0.8) (drill 0.4) (layers F.Cu B.Cu) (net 17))
 (segment (start 115.375001 90.689999) (end 115.375001 97.524999) (width 0.25) (layer B.Cu) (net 17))
 (segment (start 115.310001 90.624999) (end 115.375001 90.689999) (width 0.25) (layer B.Cu) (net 17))
 (segment (start 115.375001 97.524999) (end 111.6 101.3) (width 0.25) (layer B.Cu) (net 17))
 (segment (start 111.6 102.825) (end 111.375 103.05) (width 0.25) (layer F.Cu) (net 17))
 (segment (start 111.6 101.3) (end 111.6 102.825) (width 0.25) (layer F.Cu) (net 17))
 (segment (start 115.310001 90.370001) (end 114.2 89.26) (width 0.25) (layer B.Cu) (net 17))
 (segment (start 115.310001 90.624999) (end 115.310001 90.370001) (width 0.25) (layer B.Cu) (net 17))
 (segment (start 103.815002 81.774998) (end 101.76 83.83) (width 0.25) (layer F.Cu) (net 25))
 (segment (start 105.448002 81.774998) (end 103.815002 81.774998) (width 0.25) (layer F.Cu) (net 25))
 (segment (start 110.11 83.83) (end 107.503004 83.83) (width 0.25) (layer F.Cu) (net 25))
 (segment (start 101.76 83.83) (end 100.71 83.83) (width 0.25) (layer F.Cu) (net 25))
 (segment (start 107.503004 83.83) (end 105.448002 81.774998) (width 0.25) (layer F.Cu) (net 25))
 (segment (start 100.2 99.3375) (end 101 99.3375) (width 0.25) (layer F.Cu) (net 25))
 (segment (start 101.21 96.38) (end 101.21 95.33) (width 0.25) (layer F.Cu) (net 25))
 (segment (start 101 99.3375) (end 102.025001 98.312499) (width 0.25) (layer F.Cu) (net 25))
 (segment (start 102.025001 97.195001) (end 101.21 96.38) (width 0.25) (layer F.Cu) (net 25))
 (segment (start 108.89 97.1) (end 104 97.1) (width 0.25) (layer F.Cu) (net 25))
 (via (at 104 97.1) (size 0.8) (drill 0.4) (layers F.Cu B.Cu) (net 25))
 (via (at 102.025001 97.9) (size 0.8) (drill 0.4) (layers F.Cu B.Cu) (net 25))
 (segment (start 102.825001 97.1) (end 102.025001 97.9) (width 0.25) (layer B.Cu) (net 25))
 (segment (start 104 97.1) (end 102.825001 97.1) (width 0.25) (layer B.Cu) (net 25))
 (segment (start 102.025001 98.312499) (end 102.025001 97.9) (width 0.25) (layer F.Cu) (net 25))
 (segment (start 102.025001 97.9) (end 102.025001 97.195001) (width 0.25) (layer F.Cu) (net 25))
 (segment (start 110.11 83.38896) (end 110.11 83.83) (width 0.25) (layer F.Cu) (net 25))
 (segment (start 109.61 96.38) (end 109.61 95.33) (width 0.25) (layer F.Cu) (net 25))
 (segment (start 110.06 95.33) (end 109.61 95.33) (width 0.25) (layer F.Cu) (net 25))
 (segment (start 111.77 95.33) (end 110.06 95.33) (width 0.25) (layer F.Cu) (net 25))
 (segment (start 114.2 92.9) (end 111.77 95.33) (width 0.25) (layer F.Cu) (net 25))
 (segment (start 114.2 91.8) (end 114.2 92.9) (width 0.25) (layer F.Cu) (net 25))
 (segment (start 112.09896 81.4) (end 113.5 81.4) (width 0.25) (layer F.Cu) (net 25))
 (segment (start 110.11 83.38896) (end 112.09896 81.4) (width 0.25) (layer F.Cu) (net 25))
 (segment (start 115.375001 91.724999) (end 115.3 91.8) (width 0.25) (layer F.Cu) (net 25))
 (segment (start 114.10104 81.4) (end 115.375001 82.673961) (width 0.25) (layer F.Cu) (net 25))
 (segment (start 115.3 91.8) (end 114.2 91.8) (width 0.25) (layer F.Cu) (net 25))
 (segment (start 115.375001 82.673961) (end 115.375001 91.724999) (width 0.25) (layer F.Cu) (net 25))
 (segment (start 113.5 81.4) (end 114.10104 81.4) (width 0.25) (layer F.Cu) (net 25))
 (via (at 111.5 96.8) (size 0.8) (drill 0.4) (layers F.Cu B.Cu) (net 25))
 (segment (start 114.2 94.1) (end 111.5 96.8) (width 0.25) (layer B.Cu) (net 25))
 (segment (start 114.2 91.8) (end 114.2 94.1) (width 0.25) (layer B.Cu) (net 25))
 (segment (start 109.39 96.6) (end 108.89 97.1) (width 0.25) (layer F.Cu) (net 25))
 (segment (start 109.61 96.38) (end 109.39 96.6) (width 0.25) (layer F.Cu) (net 25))
 (segment (start 111.5 96.8) (end 111 97.3) (width 0.25) (layer F.Cu) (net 25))
 (segment (start 109.09 97.3) (end 108.89 97.1) (width 0.25) (layer F.Cu) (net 25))
 (segment (start 111 97.3) (end 109.09 97.3) (width 0.25) (layer F.Cu) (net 25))
 (segment (start 101.91 96.135) (end 101.91 95.33) (width 0.25) (layer F.Cu) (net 26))
 (segment (start 103.425 97.65) (end 101.91 96.135) (width 0.25) (layer F.Cu) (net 26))
 (segment (start 103.425 98.55) (end 103.425 97.65) (width 0.25) (layer F.Cu) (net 26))
 (segment (start 104.45 98.55) (end 111.375 98.55) (width 0.25) (layer F.Cu) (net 26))
 (segment (start 103.425 98.55) (end 104.45 98.55) (width 0.25) (layer F.Cu) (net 26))
 (segment (start 111.137341 85.337339) (end 111.53734 84.93734) (width 0.25) (layer F.Cu) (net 19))
 (via (at 111.53734 84.93734) (size 0.8) (drill 0.4) (layers F.Cu B.Cu) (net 19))
 (segment (start 110.11 85.43) (end 111.04468 85.43) (width 0.25) (layer F.Cu) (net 19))
 (segment (start 111.04468 85.43) (end 111.137341 85.337339) (width 0.25) (layer F.Cu) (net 19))
 (segment (start 113.5 84.4) (end 112.07468 84.4) (width 0.25) (layer B.Cu) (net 19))
 (segment (start 112.07468 84.4) (end 111.53734 84.93734) (width 0.25) (layer B.Cu) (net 19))
 (segment (start 111.849999 86.150001) (end 111.8 86.2) (width 0.25) (layer B.Cu) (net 20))
 (segment (start 114.185001 86.150001) (end 111.849999 86.150001) (width 0.25) (layer B.Cu) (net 20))
 (segment (start 114.250001 86.085001) (end 114.185001 86.150001) (width 0.25) (layer B.Cu) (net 20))
 (segment (start 114.250001 84.039999) (end 114.250001 86.085001) (width 0.25) (layer B.Cu) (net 20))
 (segment (start 113.139999 83.649999) (end 113.860001 83.649999) (width 0.25) (layer B.Cu) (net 20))
 (segment (start 113.389998 83.4) (end 113.139999 83.649999) (width 0.25) (layer B.Cu) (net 20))
 (segment (start 113.5 83.4) (end 113.389998 83.4) (width 0.25) (layer B.Cu) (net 20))
 (via (at 111.8 86.2) (size 0.8) (drill 0.4) (layers F.Cu B.Cu) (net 20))
 (segment (start 113.860001 83.649999) (end 114.250001 84.039999) (width 0.25) (layer B.Cu) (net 20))
 (segment (start 110.18 86.2) (end 110.11 86.13) (width 0.25) (layer F.Cu) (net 20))
 (segment (start 111.8 86.2) (end 110.18 86.2) (width 0.25) (layer F.Cu) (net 20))
 (segment (start 113.5 82.4) (end 112.89896 82.4) (width 0.25) (layer F.Cu) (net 21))
 (segment (start 111.455001 87.125001) (end 111.16 86.83) (width 0.25) (layer F.Cu) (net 21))
 (segment (start 111.948001 87.125001) (end 111.455001 87.125001) (width 0.25) (layer F.Cu) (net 21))
 (segment (start 112.525001 86.548001) (end 111.948001 87.125001) (width 0.25) (layer F.Cu) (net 21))
 (segment (start 111.16 86.83) (end 110.11 86.83) (width 0.25) (layer F.Cu) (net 21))
 (segment (start 112.525001 82.773959) (end 112.525001 86.548001) (width 0.25) (layer F.Cu) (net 21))
 (segment (start 112.89896 82.4) (end 112.525001 82.773959) (width 0.25) (layer F.Cu) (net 21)))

